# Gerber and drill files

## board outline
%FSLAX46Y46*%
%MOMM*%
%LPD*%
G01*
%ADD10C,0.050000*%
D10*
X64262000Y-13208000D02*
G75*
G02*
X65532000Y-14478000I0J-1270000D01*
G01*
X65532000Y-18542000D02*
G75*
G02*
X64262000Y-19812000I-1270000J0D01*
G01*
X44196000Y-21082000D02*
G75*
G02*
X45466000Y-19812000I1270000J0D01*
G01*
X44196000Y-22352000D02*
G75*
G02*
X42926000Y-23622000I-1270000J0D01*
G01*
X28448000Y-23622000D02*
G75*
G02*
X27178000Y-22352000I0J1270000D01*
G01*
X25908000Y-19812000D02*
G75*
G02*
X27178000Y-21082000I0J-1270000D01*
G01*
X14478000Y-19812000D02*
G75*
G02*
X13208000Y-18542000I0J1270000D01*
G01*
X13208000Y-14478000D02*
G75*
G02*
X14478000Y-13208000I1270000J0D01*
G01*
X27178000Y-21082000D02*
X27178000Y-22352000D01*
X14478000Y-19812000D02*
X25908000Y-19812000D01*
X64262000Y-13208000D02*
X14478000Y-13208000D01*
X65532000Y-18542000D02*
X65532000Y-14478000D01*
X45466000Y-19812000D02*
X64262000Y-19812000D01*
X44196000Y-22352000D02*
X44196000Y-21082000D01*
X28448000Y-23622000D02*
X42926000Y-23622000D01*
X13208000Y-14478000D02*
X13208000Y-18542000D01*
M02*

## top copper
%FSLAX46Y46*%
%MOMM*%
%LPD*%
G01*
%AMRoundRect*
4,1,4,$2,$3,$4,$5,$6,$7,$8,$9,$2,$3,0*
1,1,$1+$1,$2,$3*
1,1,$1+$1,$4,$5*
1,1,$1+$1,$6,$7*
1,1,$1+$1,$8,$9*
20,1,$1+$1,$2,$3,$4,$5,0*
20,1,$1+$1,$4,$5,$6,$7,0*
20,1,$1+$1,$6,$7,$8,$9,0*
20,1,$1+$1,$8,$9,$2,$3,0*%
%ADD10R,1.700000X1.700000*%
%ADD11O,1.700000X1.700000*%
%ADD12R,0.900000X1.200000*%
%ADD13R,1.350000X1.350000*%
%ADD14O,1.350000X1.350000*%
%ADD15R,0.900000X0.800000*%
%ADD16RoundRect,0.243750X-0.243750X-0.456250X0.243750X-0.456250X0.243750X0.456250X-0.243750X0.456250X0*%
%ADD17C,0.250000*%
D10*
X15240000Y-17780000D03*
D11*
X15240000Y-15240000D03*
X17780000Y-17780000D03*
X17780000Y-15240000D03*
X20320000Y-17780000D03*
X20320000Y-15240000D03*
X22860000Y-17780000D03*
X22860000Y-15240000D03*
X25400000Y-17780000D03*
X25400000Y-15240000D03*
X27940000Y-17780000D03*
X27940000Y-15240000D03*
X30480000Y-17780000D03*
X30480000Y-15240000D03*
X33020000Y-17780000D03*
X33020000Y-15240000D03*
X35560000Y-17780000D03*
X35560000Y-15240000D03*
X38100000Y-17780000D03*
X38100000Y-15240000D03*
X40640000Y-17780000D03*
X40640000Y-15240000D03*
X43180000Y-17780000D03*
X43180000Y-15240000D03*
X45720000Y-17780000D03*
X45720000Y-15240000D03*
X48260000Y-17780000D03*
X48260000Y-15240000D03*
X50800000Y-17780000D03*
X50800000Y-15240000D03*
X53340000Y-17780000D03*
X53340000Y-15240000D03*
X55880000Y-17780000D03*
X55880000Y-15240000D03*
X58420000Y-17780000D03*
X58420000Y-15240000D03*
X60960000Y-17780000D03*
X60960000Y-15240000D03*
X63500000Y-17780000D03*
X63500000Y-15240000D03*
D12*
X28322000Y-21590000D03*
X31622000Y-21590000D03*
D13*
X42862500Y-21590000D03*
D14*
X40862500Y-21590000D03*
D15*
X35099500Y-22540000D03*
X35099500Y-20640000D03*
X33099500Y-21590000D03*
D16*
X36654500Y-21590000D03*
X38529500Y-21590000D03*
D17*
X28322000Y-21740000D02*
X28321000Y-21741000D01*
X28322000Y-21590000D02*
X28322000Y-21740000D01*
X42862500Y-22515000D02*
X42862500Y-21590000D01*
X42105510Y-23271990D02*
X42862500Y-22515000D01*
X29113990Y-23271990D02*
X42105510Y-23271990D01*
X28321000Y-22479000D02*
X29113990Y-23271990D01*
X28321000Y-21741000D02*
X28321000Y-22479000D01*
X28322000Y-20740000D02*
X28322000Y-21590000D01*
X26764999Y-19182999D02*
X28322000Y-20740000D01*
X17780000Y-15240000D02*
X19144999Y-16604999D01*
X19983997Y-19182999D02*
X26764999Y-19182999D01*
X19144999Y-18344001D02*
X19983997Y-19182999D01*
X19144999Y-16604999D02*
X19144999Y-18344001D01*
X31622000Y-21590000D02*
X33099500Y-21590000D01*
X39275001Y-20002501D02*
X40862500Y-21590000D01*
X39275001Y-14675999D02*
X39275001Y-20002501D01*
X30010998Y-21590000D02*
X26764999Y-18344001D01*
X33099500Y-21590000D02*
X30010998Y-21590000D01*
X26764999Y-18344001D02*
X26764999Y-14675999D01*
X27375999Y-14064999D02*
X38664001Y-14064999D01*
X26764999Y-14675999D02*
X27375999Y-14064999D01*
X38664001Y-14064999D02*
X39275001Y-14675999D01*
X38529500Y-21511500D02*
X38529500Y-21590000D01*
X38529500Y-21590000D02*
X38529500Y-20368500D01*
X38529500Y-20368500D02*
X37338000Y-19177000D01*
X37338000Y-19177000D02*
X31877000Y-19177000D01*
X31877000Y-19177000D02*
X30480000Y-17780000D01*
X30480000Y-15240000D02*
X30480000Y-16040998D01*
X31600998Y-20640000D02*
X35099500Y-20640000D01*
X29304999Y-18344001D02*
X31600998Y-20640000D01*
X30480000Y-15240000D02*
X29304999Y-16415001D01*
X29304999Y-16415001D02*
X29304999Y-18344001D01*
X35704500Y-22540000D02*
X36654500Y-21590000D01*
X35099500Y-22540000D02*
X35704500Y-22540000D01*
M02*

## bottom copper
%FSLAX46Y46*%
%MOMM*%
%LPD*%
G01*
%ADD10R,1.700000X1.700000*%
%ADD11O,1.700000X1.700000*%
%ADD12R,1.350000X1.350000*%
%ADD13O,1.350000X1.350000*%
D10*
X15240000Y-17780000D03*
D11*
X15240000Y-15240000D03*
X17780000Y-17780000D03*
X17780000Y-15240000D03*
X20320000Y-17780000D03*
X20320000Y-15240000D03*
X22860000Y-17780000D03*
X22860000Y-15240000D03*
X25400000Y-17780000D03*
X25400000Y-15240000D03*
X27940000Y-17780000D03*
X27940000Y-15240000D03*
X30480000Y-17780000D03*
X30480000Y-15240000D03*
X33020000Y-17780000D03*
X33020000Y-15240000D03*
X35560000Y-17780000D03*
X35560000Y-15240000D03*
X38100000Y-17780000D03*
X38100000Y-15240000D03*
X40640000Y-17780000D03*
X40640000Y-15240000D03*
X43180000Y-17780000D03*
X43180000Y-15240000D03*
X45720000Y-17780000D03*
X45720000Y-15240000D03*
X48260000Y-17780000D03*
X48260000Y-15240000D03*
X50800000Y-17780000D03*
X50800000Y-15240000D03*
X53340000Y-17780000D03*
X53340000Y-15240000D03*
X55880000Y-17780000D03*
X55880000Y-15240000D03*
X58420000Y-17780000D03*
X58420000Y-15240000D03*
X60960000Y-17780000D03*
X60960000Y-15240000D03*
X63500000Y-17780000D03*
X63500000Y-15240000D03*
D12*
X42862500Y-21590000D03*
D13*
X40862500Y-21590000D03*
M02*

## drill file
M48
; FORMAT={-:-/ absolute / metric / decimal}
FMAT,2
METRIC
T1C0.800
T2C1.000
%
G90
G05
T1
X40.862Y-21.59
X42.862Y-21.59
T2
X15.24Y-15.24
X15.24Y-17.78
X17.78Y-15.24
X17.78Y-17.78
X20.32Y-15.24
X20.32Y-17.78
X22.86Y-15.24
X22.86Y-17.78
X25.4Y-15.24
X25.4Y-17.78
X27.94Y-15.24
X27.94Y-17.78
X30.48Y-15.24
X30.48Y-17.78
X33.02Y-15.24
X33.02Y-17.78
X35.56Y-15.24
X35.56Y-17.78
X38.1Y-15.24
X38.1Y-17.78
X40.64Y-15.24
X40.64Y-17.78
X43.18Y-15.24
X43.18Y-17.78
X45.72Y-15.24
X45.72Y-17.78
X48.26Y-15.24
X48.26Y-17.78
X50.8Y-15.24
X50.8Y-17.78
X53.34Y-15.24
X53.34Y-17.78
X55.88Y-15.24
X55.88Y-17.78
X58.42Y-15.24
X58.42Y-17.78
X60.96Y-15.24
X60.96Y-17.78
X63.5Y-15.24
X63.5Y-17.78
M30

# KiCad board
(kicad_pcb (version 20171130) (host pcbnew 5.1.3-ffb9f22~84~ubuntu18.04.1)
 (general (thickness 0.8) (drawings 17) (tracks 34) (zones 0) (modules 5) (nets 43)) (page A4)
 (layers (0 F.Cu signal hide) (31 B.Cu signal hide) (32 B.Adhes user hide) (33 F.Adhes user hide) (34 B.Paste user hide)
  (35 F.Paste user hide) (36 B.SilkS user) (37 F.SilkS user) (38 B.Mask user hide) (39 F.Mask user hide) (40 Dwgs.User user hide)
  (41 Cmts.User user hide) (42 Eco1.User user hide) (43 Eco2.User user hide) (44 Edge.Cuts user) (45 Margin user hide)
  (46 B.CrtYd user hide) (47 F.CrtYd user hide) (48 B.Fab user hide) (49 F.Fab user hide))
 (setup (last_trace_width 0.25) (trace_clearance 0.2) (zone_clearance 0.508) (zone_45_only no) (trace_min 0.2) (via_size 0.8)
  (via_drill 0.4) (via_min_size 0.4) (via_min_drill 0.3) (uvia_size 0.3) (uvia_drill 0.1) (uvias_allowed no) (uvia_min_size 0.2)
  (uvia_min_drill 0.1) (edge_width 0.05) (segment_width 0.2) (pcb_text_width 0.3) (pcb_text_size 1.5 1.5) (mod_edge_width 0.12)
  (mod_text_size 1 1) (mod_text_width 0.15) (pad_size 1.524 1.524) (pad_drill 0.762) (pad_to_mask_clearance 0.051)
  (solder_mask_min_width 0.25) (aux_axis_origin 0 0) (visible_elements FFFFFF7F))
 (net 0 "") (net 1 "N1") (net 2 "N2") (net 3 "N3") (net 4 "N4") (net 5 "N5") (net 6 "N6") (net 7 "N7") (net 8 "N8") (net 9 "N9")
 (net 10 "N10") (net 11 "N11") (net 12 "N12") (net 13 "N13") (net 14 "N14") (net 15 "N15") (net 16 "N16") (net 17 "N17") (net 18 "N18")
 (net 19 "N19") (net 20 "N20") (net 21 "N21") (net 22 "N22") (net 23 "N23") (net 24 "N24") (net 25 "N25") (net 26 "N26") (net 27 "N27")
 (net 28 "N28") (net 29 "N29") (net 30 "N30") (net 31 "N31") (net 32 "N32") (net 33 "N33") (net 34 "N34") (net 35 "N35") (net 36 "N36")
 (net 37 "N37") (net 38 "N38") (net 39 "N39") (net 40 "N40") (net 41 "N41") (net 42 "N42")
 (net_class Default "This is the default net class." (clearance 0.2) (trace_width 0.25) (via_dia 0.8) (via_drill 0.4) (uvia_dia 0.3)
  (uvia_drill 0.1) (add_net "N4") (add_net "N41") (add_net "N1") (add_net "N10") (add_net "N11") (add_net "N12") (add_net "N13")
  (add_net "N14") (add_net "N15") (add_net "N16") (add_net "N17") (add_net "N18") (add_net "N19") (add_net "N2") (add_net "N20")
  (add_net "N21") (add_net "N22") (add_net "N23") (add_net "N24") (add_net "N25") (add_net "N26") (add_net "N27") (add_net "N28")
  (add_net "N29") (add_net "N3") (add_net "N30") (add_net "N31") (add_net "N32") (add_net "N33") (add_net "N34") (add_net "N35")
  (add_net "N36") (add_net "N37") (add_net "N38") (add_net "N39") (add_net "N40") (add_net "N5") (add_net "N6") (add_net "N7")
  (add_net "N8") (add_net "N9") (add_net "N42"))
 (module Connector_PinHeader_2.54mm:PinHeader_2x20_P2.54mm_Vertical (layer F.Cu) (at 15.24 17.78 90)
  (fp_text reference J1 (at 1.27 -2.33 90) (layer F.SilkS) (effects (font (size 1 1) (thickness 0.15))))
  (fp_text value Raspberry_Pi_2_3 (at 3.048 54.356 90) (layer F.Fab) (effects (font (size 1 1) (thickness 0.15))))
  (pad 1 thru_hole rect (at 0 0 90) (size 1.7 1.7) (drill 1) (layers *.Cu *.Mask) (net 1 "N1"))
  (pad 2 thru_hole oval (at 2.54 0 90) (size 1.7 1.7) (drill 1) (layers *.Cu *.Mask) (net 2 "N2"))
  (pad 3 thru_hole oval (at 0 2.54 90) (size 1.7 1.7) (drill 1) (layers *.Cu *.Mask) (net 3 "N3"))
  (pad 4 thru_hole oval (at 2.54 2.54 90) (size 1.7 1.7) (drill 1) (layers *.Cu *.Mask) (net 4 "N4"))
  (pad 5 thru_hole oval (at 0 5.08 90) (size 1.7 1.7) (drill 1) (layers *.Cu *.Mask) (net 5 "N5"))
  (pad 6 thru_hole oval (at 2.54 5.08 90) (size 1.7 1.7) (drill 1) (layers *.Cu *.Mask) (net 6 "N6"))
  (pad 7 thru_hole oval (at 0 7.62 90) (size 1.7 1.7) (drill 1) (layers *.Cu *.Mask) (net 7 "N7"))
  (pad 8 thru_hole oval (at 2.54 7.62 90) (size 1.7 1.7) (drill 1) (layers *.Cu *.Mask) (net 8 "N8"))
  (pad 9 thru_hole oval (at 0 10.16 90) (size 1.7 1.7) (drill 1) (layers *.Cu *.Mask) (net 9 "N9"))
  (pad 10 thru_hole oval (at 2.54 10.16 90) (size 1.7 1.7) (drill 1) (layers *.Cu *.Mask) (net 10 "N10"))
  (pad 11 thru_hole oval (at 0 12.7 90) (size 1.7 1.7) (drill 1) (layers *.Cu *.Mask) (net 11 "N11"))
  (pad 12 thru_hole oval (at 2.54 12.7 90) (size 1.7 1.7) (drill 1) (layers *.Cu *.Mask) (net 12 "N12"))
  (pad 13 thru_hole oval (at 0 15.24 90) (size 1.7 1.7) (drill 1) (layers *.Cu *.Mask) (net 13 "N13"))
  (pad 14 thru_hole oval (at 2.54 15.24 90) (size 1.7 1.7) (drill 1) (layers *.Cu *.Mask) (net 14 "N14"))
  (pad 15 thru_hole oval (at 0 17.78 90) (size 1.7 1.7) (drill 1) (layers *.Cu *.Mask) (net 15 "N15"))
  (pad 16 thru_hole oval (at 2.54 17.78 90) (size 1.7 1.7) (drill 1) (layers *.Cu *.Mask) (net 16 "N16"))
  (pad 17 thru_hole oval (at 0 20.32 90) (size 1.7 1.7) (drill 1) (layers *.Cu *.Mask) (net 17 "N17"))
  (pad 18 thru_hole oval (at 2.54 20.32 90) (size 1.7 1.7) (drill 1) (layers *.Cu *.Mask) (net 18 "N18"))
  (pad 19 thru_hole oval (at 0 22.86 90) (size 1.7 1.7) (drill 1) (layers *.Cu *.Mask) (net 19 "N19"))
  (pad 20 thru_hole oval (at 2.54 22.86 90) (size 1.7 1.7) (drill 1) (layers *.Cu *.Mask) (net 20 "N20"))
  (pad 21 thru_hole oval (at 0 25.4 90) (size 1.7 1.7) (drill 1) (layers *.Cu *.Mask) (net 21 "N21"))
  (pad 22 thru_hole oval (at 2.54 25.4 90) (size 1.7 1.7) (drill 1) (layers *.Cu *.Mask) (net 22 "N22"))
  (pad 23 thru_hole oval (at 0 27.94 90) (size 1.7 1.7) (drill 1) (layers *.Cu *.Mask) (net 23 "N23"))
  (pad 24 thru_hole oval (at 2.54 27.94 90) (size 1.7 1.7) (drill 1) (layers *.Cu *.Mask) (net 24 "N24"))
  (pad 25 thru_hole oval (at 0 30.48 90) (size 1.7 1.7) (drill 1) (layers *.Cu *.Mask) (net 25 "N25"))
  (pad 26 thru_hole oval (at 2.54 30.48 90) (size 1.7 1.7) (drill 1) (layers *.Cu *.Mask) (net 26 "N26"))
  (pad 27 thru_hole oval (at 0 33.02 90) (size 1.7 1.7) (drill 1) (layers *.Cu *.Mask) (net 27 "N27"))
  (pad 28 thru_hole oval (at 2.54 33.02 90) (size 1.7 1.7) (drill 1) (layers *.Cu *.Mask) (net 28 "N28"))
  (pad 29 thru_hole oval (at 0 35.56 90) (size 1.7 1.7) (drill 1) (layers *.Cu *.Mask) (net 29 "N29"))
  (pad 30 thru_hole oval (at 2.54 35.56 90) (size 1.7 1.7) (drill 1) (layers *.Cu *.Mask) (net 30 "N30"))
  (pad 31 thru_hole oval (at 0 38.1 90) (size 1.7 1.7) (drill 1) (layers *.Cu *.Mask) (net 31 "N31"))
  (pad 32 thru_hole oval (at 2.54 38.1 90) (size 1.7 1.7) (drill 1) (layers *.Cu *.Mask) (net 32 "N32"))
  (pad 33 thru_hole oval (at 0 40.64 90) (size 1.7 1.7) (drill 1) (layers *.Cu *.Mask) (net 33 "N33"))
  (pad 34 thru_hole oval (at 2.54 40.64 90) (size 1.7 1.7) (drill 1) (layers *.Cu *.Mask) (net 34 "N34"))
  (pad 35 thru_hole oval (at 0 43.18 90) (size 1.7 1.7) (drill 1) (layers *.Cu *.Mask) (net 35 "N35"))
  (pad 36 thru_hole oval (at 2.54 43.18 90) (size 1.7 1.7) (drill 1) (layers *.Cu *.Mask) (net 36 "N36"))
  (pad 37 thru_hole oval (at 0 45.72 90) (size 1.7 1.7) (drill 1) (layers *.Cu *.Mask) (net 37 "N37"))
  (pad 38 thru_hole oval (at 2.54 45.72 90) (size 1.7 1.7) (drill 1) (layers *.Cu *.Mask) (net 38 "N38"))
  (pad 39 thru_hole oval (at 0 48.26 90) (size 1.7 1.7) (drill 1) (layers *.Cu *.Mask) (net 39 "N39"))
  (pad 40 thru_hole oval (at 2.54 48.26 90) (size 1.7 1.7) (drill 1) (layers *.Cu *.Mask) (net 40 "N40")))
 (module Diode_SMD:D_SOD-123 (layer F.Cu) (at 29.972 21.59)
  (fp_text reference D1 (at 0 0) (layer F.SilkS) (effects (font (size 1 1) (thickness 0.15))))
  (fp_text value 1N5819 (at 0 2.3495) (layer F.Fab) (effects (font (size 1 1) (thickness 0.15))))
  (pad 1 smd rect (at -1.65 0) (size 0.9 1.2) (layers F.Cu F.Paste F.Mask) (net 4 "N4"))
  (pad 2 smd rect (at 1.65 0) (size 0.9 1.2) (layers F.Cu F.Paste F.Mask) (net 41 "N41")))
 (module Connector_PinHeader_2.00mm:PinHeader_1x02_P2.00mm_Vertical (layer F.Cu) (at 42.8625 21.59 270)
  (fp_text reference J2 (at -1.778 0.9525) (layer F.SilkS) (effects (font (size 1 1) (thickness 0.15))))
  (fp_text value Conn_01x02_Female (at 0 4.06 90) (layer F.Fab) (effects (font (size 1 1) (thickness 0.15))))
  (pad 1 thru_hole rect (at 0 0 270) (size 1.35 1.35) (drill 0.8) (layers *.Cu *.Mask) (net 4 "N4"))
  (pad 2 thru_hole oval (at 0 2 270) (size 1.35 1.35) (drill 0.8) (layers *.Cu *.Mask) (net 41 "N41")))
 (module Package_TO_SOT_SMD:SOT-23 (layer F.Cu) (at 34.0995 21.59 180)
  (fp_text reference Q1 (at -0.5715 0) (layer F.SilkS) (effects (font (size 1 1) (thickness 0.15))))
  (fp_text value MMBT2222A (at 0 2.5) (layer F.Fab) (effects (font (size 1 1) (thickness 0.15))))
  (pad 1 smd rect (at -1 -0.95 180) (size 0.9 0.8) (layers F.Cu F.Paste F.Mask) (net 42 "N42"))
  (pad 2 smd rect (at -1 0.95 180) (size 0.9 0.8) (layers F.Cu F.Paste F.Mask) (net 14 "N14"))
  (pad 3 smd rect (at 1 0 180) (size 0.9 0.8) (layers F.Cu F.Paste F.Mask) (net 41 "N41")))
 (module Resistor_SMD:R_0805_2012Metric (layer F.Cu) (at 37.592 21.59)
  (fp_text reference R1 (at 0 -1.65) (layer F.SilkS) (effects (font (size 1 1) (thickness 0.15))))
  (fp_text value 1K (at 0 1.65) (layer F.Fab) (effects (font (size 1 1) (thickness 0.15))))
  (pad 1 smd roundrect (at -0.9375 0) (size 0.975 1.4) (layers F.Cu F.Paste F.Mask) (roundrect_rratio 0.25) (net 42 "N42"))
  (pad 2 smd roundrect (at 0.9375 0) (size 0.975 1.4) (layers F.Cu F.Paste F.Mask) (roundrect_rratio 0.25) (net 13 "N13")))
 (gr_arc (start 64.262 14.478) (end 65.532 14.478) (angle -90) (layer Edge.Cuts) (width 0.05))
 (gr_arc (start 64.262 18.542) (end 64.262 19.812) (angle -90) (layer Edge.Cuts) (width 0.05))
 (gr_arc (start 45.466 21.082) (end 45.466 19.812) (angle -90) (layer Edge.Cuts) (width 0.05))
 (gr_arc (start 42.926 22.352) (end 42.926 23.622) (angle -90) (layer Edge.Cuts) (width 0.05))
 (gr_arc (start 28.448 22.352) (end 27.178 22.352) (angle -90) (layer Edge.Cuts) (width 0.05))
 (gr_arc (start 25.908 21.082) (end 27.178 21.082) (angle -90) (layer Edge.Cuts) (width 0.05))
 (gr_arc (start 14.478 18.542) (end 13.208 18.542) (angle -90) (layer Edge.Cuts) (width 0.05))
 (gr_arc (start 14.478 14.478) (end 14.478 13.208) (angle -90) (layer Edge.Cuts) (width 0.05))
 (gr_line (start 27.178 21.082) (end 27.178 22.352) (layer Edge.Cuts) (width 0.05))
 (gr_line (start 14.478 19.812) (end 25.908 19.812) (layer Edge.Cuts) (width 0.05))
 (gr_line (start 64.262 13.208) (end 14.478 13.208) (layer Edge.Cuts) (width 0.05))
 (gr_line (start 65.532 18.542) (end 65.532 14.478) (layer Edge.Cuts) (width 0.05))
 (gr_line (start 45.466 19.812) (end 64.262 19.812) (layer Edge.Cuts) (width 0.05))
 (gr_line (start 44.196 22.352) (end 44.196 21.082) (layer Edge.Cuts) (width 0.05))
 (gr_line (start 28.448 23.622) (end 42.926 23.622) (layer Edge.Cuts) (width 0.05))
 (gr_line (start 13.208 14.478) (end 13.208 18.542) (layer Edge.Cuts) (width 0.05))
 (segment (start 28.322 21.74) (end 28.321 21.741) (width 0.25) (layer F.Cu) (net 4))
 (segment (start 28.322 21.59) (end 28.322 21.74) (width 0.25) (layer F.Cu) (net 4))
 (segment (start 42.8625 22.515) (end 42.8625 21.59) (width 0.25) (layer F.Cu) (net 4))
 (segment (start 42.10551 23.27199) (end 42.8625 22.515) (width 0.25) (layer F.Cu) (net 4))
 (segment (start 29.11399 23.27199) (end 42.10551 23.27199) (width 0.25) (layer F.Cu) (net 4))
 (segment (start 28.321 22.479) (end 29.11399 23.27199) (width 0.25) (layer F.Cu) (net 4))
 (segment (start 28.321 21.741) (end 28.321 22.479) (width 0.25) (layer F.Cu) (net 4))
 (segment (start 28.322 20.74) (end 28.322 21.59) (width 0.25) (layer F.Cu) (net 4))
 (segment (start 26.764999 19.182999) (end 28.322 20.74) (width 0.25) (layer F.Cu) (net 4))
 (segment (start 17.78 15.24) (end 19.144999 16.604999) (width 0.25) (layer F.Cu) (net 4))
 (segment (start 19.983997 19.182999) (end 26.764999 19.182999) (width 0.25) (layer F.Cu) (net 4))
 (segment (start 19.144999 18.344001) (end 19.983997 19.182999) (width 0.25) (layer F.Cu) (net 4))
 (segment (start 19.144999 16.604999) (end 19.144999 18.344001) (width 0.25) (layer F.Cu) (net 4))
 (segment (start 31.622 21.59) (end 33.0995 21.59) (width 0.25) (layer F.Cu) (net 41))
 (segment (start 39.275001 20.002501) (end 40.8625 21.59) (width 0.25) (layer F.Cu) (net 41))
 (segment (start 39.275001 14.675999) (end 39.275001 20.002501) (width 0.25) (layer F.Cu) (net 41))
 (segment (start 30.010998 21.59) (end 26.764999 18.344001) (width 0.25) (layer F.Cu) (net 41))
 (segment (start 33.0995 21.59) (end 30.010998 21.59) (width 0.25) (layer F.Cu) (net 41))
 (segment (start 26.764999 18.344001) (end 26.764999 14.675999) (width 0.25) (layer F.Cu) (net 41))
 (segment (start 27.375999 14.064999) (end 38.664001 14.064999) (width 0.25) (layer F.Cu) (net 41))
 (segment (start 26.764999 14.675999) (end 27.375999 14.064999) (width 0.25) (layer F.Cu) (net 41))
 (segment (start 38.664001 14.064999) (end 39.275001 14.675999) (width 0.25) (layer F.Cu) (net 41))
 (segment (start 38.5295 21.5115) (end 38.5295 21.59) (width 0.25) (layer F.Cu) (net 13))
 (segment (start 38.5295 21.59) (end 38.5295 20.3685) (width 0.25) (layer F.Cu) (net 13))
 (segment (start 38.5295 20.3685) (end 37.338 19.177) (width 0.25) (layer F.Cu) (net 13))
 (segment (start 37.338 19.177) (end 31.877 19.177) (width 0.25) (layer F.Cu) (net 13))
 (segment (start 31.877 19.177) (end 30.48 17.78) (width 0.25) (layer F.Cu) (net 13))
 (segment (start 30.48 15.24) (end 30.48 16.040998) (width 0.25) (layer F.Cu) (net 14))
 (segment (start 31.600998 20.64) (end 35.0995 20.64) (width 0.25) (layer F.Cu) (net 14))
 (segment (start 29.304999 18.344001) (end 31.600998 20.64) (width 0.25) (layer F.Cu) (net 14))
 (segment (start 30.48 15.24) (end 29.304999 16.415001) (width 0.25) (layer F.Cu) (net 14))
 (segment (start 29.304999 16.415001) (end 29.304999 18.344001) (width 0.25) (layer F.Cu) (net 14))
 (segment (start 35.7045 22.54) (end 36.6545 21.59) (width 0.25) (layer F.Cu) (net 42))
 (segment (start 35.0995 22.54) (end 35.7045 22.54) (width 0.25) (layer F.Cu) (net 42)))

